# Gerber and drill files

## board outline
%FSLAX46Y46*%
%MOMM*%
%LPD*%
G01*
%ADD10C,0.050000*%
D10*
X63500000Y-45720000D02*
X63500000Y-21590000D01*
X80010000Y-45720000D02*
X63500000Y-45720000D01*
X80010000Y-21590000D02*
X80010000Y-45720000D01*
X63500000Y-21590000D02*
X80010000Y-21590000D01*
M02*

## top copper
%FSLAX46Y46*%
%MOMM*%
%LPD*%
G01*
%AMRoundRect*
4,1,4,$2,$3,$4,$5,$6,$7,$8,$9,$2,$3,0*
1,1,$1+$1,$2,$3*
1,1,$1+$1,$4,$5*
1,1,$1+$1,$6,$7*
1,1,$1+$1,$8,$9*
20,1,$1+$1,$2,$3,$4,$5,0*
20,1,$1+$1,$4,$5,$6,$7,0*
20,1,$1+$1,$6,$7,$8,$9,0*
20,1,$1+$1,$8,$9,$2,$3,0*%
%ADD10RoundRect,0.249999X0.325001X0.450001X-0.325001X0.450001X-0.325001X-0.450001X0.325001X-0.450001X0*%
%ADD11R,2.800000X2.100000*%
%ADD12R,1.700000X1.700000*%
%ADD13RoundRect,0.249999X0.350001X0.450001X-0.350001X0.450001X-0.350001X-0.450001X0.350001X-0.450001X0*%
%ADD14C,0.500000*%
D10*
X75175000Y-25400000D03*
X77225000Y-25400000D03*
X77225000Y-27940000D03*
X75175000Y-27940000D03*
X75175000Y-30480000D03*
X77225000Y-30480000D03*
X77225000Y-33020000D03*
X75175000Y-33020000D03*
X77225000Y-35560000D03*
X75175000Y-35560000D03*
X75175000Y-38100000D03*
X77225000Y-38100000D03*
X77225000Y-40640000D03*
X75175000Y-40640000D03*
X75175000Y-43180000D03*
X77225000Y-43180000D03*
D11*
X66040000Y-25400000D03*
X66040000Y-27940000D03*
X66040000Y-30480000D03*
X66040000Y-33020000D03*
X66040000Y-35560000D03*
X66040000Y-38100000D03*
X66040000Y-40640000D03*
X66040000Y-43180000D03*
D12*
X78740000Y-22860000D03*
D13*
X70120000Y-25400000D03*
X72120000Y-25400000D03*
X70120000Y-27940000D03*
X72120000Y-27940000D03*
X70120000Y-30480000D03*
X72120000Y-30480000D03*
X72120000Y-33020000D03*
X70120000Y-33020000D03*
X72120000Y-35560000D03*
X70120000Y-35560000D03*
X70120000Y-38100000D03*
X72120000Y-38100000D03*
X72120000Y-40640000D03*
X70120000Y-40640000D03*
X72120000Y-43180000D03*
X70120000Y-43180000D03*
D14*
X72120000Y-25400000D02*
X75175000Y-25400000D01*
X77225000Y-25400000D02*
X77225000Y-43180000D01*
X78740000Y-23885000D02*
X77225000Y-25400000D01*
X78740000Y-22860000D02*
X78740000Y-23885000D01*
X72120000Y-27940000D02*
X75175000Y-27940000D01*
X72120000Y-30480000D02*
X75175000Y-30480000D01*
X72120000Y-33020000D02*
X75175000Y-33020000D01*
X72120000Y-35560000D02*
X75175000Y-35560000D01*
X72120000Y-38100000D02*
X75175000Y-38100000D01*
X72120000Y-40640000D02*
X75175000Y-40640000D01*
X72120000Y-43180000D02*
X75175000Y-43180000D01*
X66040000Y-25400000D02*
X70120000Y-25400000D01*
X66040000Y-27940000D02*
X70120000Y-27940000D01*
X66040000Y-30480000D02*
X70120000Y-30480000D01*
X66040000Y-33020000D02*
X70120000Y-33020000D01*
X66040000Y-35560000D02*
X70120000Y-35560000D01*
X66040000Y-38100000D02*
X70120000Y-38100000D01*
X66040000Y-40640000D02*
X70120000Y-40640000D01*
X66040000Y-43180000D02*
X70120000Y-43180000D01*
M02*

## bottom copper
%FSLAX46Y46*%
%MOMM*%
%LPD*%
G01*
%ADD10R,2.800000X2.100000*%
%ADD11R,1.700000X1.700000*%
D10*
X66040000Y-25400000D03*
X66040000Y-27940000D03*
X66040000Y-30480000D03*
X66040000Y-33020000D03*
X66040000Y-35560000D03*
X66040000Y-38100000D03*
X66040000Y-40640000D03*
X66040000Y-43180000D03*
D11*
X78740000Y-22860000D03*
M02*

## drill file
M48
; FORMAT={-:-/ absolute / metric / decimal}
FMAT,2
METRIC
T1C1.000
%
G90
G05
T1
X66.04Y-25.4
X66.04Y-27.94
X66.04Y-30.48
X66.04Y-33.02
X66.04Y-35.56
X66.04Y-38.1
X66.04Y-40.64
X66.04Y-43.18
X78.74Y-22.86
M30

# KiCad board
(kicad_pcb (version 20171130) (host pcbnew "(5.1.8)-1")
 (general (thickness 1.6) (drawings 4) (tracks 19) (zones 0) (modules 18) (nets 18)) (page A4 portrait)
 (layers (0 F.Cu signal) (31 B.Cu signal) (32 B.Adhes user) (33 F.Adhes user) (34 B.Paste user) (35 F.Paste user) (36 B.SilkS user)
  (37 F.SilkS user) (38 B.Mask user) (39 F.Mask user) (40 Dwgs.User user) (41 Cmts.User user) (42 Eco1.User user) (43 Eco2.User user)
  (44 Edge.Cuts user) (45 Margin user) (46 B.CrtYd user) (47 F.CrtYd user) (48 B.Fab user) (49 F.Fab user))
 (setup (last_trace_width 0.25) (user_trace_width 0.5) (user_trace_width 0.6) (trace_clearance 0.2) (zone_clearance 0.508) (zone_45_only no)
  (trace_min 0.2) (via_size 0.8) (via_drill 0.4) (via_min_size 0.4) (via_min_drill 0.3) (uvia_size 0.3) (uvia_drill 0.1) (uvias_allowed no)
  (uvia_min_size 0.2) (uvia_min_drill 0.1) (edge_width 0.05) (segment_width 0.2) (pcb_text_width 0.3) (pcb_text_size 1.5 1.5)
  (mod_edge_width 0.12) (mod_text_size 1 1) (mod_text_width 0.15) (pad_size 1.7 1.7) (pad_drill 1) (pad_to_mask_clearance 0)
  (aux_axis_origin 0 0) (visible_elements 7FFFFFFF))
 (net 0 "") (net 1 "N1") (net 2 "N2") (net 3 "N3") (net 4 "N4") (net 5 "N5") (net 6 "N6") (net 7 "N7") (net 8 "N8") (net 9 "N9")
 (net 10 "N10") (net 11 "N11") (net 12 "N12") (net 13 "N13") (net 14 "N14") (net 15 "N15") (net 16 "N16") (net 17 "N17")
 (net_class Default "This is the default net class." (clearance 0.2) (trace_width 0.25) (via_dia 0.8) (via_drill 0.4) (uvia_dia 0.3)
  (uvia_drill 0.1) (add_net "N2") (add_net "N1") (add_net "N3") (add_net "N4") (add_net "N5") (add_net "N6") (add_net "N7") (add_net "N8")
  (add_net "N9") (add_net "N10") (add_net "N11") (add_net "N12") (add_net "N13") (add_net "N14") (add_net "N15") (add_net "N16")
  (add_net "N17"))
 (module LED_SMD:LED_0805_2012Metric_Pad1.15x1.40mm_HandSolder (layer F.Cu) (at 76.2 25.4 180)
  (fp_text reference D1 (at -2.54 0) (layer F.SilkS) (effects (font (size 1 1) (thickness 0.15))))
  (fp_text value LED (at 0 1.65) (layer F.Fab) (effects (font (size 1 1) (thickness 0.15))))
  (pad 2 smd roundrect (at 1.025 0 180) (size 1.15 1.4) (layers F.Cu F.Paste F.Mask) (roundrect_rratio 0.2173904347826087) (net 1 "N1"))
  (pad 1 smd roundrect (at -1.025 0 180) (size 1.15 1.4) (layers F.Cu F.Paste F.Mask) (roundrect_rratio 0.2173904347826087) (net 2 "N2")))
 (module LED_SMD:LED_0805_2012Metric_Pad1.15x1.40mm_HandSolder (layer F.Cu) (at 76.2 27.94 180)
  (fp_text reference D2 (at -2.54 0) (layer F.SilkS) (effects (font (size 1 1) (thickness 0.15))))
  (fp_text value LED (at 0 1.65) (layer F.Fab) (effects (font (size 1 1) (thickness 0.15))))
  (pad 1 smd roundrect (at -1.025 0 180) (size 1.15 1.4) (layers F.Cu F.Paste F.Mask) (roundrect_rratio 0.2173904347826087) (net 2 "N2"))
  (pad 2 smd roundrect (at 1.025 0 180) (size 1.15 1.4) (layers F.Cu F.Paste F.Mask) (roundrect_rratio 0.2173904347826087) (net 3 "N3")))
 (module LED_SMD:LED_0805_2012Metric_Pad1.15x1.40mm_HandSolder (layer F.Cu) (at 76.2 30.48 180)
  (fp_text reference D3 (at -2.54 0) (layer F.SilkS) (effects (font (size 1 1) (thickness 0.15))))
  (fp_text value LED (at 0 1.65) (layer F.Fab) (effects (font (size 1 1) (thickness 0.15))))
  (pad 2 smd roundrect (at 1.025 0 180) (size 1.15 1.4) (layers F.Cu F.Paste F.Mask) (roundrect_rratio 0.2173904347826087) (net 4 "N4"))
  (pad 1 smd roundrect (at -1.025 0 180) (size 1.15 1.4) (layers F.Cu F.Paste F.Mask) (roundrect_rratio 0.2173904347826087) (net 2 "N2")))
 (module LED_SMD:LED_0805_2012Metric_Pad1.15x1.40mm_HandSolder (layer F.Cu) (at 76.2 33.02 180)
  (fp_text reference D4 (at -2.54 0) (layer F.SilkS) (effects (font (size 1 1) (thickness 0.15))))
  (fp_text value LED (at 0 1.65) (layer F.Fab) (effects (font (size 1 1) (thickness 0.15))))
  (pad 1 smd roundrect (at -1.025 0 180) (size 1.15 1.4) (layers F.Cu F.Paste F.Mask) (roundrect_rratio 0.2173904347826087) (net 2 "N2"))
  (pad 2 smd roundrect (at 1.025 0 180) (size 1.15 1.4) (layers F.Cu F.Paste F.Mask) (roundrect_rratio 0.2173904347826087) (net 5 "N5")))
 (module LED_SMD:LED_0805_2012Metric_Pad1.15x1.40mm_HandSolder (layer F.Cu) (at 76.2 35.56 180)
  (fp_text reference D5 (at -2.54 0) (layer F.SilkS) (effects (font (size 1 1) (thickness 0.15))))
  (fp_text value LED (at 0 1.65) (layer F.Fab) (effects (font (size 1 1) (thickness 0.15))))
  (pad 1 smd roundrect (at -1.025 0 180) (size 1.15 1.4) (layers F.Cu F.Paste F.Mask) (roundrect_rratio 0.2173904347826087) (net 2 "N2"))
  (pad 2 smd roundrect (at 1.025 0 180) (size 1.15 1.4) (layers F.Cu F.Paste F.Mask) (roundrect_rratio 0.2173904347826087) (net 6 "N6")))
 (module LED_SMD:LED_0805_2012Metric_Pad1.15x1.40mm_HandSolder (layer F.Cu) (at 76.2 38.1 180)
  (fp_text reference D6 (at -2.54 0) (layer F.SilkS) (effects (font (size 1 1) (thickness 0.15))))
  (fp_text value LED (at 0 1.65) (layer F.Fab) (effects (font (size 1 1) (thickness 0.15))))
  (pad 2 smd roundrect (at 1.025 0 180) (size 1.15 1.4) (layers F.Cu F.Paste F.Mask) (roundrect_rratio 0.2173904347826087) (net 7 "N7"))
  (pad 1 smd roundrect (at -1.025 0 180) (size 1.15 1.4) (layers F.Cu F.Paste F.Mask) (roundrect_rratio 0.2173904347826087) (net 2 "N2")))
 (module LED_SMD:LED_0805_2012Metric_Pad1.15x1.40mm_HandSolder (layer F.Cu) (at 76.2 40.64 180)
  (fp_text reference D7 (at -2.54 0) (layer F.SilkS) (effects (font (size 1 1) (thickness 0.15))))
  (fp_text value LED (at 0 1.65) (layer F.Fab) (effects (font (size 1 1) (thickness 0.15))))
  (pad 1 smd roundrect (at -1.025 0 180) (size 1.15 1.4) (layers F.Cu F.Paste F.Mask) (roundrect_rratio 0.2173904347826087) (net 2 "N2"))
  (pad 2 smd roundrect (at 1.025 0 180) (size 1.15 1.4) (layers F.Cu F.Paste F.Mask) (roundrect_rratio 0.2173904347826087) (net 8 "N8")))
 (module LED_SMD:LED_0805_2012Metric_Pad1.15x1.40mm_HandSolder (layer F.Cu) (at 76.2 43.18 180)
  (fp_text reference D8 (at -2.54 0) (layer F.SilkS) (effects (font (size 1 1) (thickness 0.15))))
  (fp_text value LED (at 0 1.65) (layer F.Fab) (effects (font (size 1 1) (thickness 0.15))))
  (pad 2 smd roundrect (at 1.025 0 180) (size 1.15 1.4) (layers F.Cu F.Paste F.Mask) (roundrect_rratio 0.2173904347826087) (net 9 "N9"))
  (pad 1 smd roundrect (at -1.025 0 180) (size 1.15 1.4) (layers F.Cu F.Paste F.Mask) (roundrect_rratio 0.2173904347826087) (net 2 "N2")))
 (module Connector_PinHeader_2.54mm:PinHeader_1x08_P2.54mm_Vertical (layer F.Cu) (at 66.04 25.4)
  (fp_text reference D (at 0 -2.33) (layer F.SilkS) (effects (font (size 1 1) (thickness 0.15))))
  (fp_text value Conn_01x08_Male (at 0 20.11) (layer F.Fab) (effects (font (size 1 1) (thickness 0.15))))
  (pad 1 thru_hole rect (at 0 0) (size 2.8 2.1) (drill 1) (layers *.Cu *.Mask) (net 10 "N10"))
  (pad 2 thru_hole rect (at 0 2.54) (size 2.8 2.1) (drill 1) (layers *.Cu *.Mask) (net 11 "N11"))
  (pad 3 thru_hole rect (at 0 5.08) (size 2.8 2.1) (drill 1) (layers *.Cu *.Mask) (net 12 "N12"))
  (pad 4 thru_hole rect (at 0 7.62) (size 2.8 2.1) (drill 1) (layers *.Cu *.Mask) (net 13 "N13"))
  (pad 5 thru_hole rect (at 0 10.16) (size 2.8 2.1) (drill 1) (layers *.Cu *.Mask) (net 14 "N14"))
  (pad 6 thru_hole rect (at 0 12.7) (size 2.8 2.1) (drill 1) (layers *.Cu *.Mask) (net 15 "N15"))
  (pad 7 thru_hole rect (at 0 15.24) (size 2.8 2.1) (drill 1) (layers *.Cu *.Mask) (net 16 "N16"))
  (pad 8 thru_hole rect (at 0 17.78) (size 2.8 2.1) (drill 1) (layers *.Cu *.Mask) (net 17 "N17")))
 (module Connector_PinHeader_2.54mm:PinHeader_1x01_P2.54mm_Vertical (layer F.Cu) (at 78.74 22.86)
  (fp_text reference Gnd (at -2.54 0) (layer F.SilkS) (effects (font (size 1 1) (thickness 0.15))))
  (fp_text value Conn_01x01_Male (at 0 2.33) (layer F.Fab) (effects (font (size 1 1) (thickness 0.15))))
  (pad 1 thru_hole rect (at 0 0) (size 1.7 1.7) (drill 1) (layers *.Cu *.Mask) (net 2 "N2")))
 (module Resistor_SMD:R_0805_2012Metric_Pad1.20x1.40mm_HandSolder (layer F.Cu) (at 71.12 25.4 180)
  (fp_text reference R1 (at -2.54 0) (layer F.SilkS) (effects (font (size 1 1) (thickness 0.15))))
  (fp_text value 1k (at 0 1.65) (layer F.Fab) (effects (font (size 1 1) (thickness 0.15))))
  (pad 2 smd roundrect (at 1 0 180) (size 1.2 1.4) (layers F.Cu F.Paste F.Mask) (roundrect_rratio 0.2083325) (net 10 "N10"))
  (pad 1 smd roundrect (at -1 0 180) (size 1.2 1.4) (layers F.Cu F.Paste F.Mask) (roundrect_rratio 0.2083325) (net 1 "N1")))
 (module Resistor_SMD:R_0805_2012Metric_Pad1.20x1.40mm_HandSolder (layer F.Cu) (at 71.12 27.94 180)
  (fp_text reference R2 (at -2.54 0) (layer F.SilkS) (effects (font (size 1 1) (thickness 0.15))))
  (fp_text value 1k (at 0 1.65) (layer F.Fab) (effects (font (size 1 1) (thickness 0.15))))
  (pad 2 smd roundrect (at 1 0 180) (size 1.2 1.4) (layers F.Cu F.Paste F.Mask) (roundrect_rratio 0.2083325) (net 11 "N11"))
  (pad 1 smd roundrect (at -1 0 180) (size 1.2 1.4) (layers F.Cu F.Paste F.Mask) (roundrect_rratio 0.2083325) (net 3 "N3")))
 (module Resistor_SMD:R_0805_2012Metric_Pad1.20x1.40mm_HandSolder (layer F.Cu) (at 71.12 30.48 180)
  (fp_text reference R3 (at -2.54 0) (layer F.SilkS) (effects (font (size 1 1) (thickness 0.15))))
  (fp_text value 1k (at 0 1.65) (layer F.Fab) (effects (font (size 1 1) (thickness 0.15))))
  (pad 2 smd roundrect (at 1 0 180) (size 1.2 1.4) (layers F.Cu F.Paste F.Mask) (roundrect_rratio 0.2083325) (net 12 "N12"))
  (pad 1 smd roundrect (at -1 0 180) (size 1.2 1.4) (layers F.Cu F.Paste F.Mask) (roundrect_rratio 0.2083325) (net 4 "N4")))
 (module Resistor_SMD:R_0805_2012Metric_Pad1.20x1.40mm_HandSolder (layer F.Cu) (at 71.12 33.02 180)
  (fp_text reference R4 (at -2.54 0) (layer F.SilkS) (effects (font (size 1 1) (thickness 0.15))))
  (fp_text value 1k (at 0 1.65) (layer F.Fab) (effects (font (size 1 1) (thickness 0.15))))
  (pad 1 smd roundrect (at -1 0 180) (size 1.2 1.4) (layers F.Cu F.Paste F.Mask) (roundrect_rratio 0.2083325) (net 5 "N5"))
  (pad 2 smd roundrect (at 1 0 180) (size 1.2 1.4) (layers F.Cu F.Paste F.Mask) (roundrect_rratio 0.2083325) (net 13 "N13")))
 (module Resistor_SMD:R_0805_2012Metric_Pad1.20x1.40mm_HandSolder (layer F.Cu) (at 71.12 35.56 180)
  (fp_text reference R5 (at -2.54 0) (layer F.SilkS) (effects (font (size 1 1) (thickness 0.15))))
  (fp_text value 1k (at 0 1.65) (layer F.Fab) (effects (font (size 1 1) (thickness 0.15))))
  (pad 1 smd roundrect (at -1 0 180) (size 1.2 1.4) (layers F.Cu F.Paste F.Mask) (roundrect_rratio 0.2083325) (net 6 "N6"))
  (pad 2 smd roundrect (at 1 0 180) (size 1.2 1.4) (layers F.Cu F.Paste F.Mask) (roundrect_rratio 0.2083325) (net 14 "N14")))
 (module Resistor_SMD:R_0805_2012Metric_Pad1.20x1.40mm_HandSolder (layer F.Cu) (at 71.12 38.1 180)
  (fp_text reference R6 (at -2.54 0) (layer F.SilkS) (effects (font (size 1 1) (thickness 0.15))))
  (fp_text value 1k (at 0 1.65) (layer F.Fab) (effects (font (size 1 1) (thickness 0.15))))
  (pad 2 smd roundrect (at 1 0 180) (size 1.2 1.4) (layers F.Cu F.Paste F.Mask) (roundrect_rratio 0.2083325) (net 15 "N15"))
  (pad 1 smd roundrect (at -1 0 180) (size 1.2 1.4) (layers F.Cu F.Paste F.Mask) (roundrect_rratio 0.2083325) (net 7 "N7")))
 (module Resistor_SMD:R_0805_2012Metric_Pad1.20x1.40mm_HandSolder (layer F.Cu) (at 71.12 40.64 180)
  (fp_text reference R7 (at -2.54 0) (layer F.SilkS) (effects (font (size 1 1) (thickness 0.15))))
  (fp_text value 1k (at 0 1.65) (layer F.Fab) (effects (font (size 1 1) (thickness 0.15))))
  (pad 1 smd roundrect (at -1 0 180) (size 1.2 1.4) (layers F.Cu F.Paste F.Mask) (roundrect_rratio 0.2083325) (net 8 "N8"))
  (pad 2 smd roundrect (at 1 0 180) (size 1.2 1.4) (layers F.Cu F.Paste F.Mask) (roundrect_rratio 0.2083325) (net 16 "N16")))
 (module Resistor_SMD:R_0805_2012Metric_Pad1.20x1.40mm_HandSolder (layer F.Cu) (at 71.12 43.18 180)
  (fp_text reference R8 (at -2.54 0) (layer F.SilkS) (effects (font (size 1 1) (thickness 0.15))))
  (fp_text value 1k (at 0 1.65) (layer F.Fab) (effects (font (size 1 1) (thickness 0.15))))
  (pad 1 smd roundrect (at -1 0 180) (size 1.2 1.4) (layers F.Cu F.Paste F.Mask) (roundrect_rratio 0.2083325) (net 9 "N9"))
  (pad 2 smd roundrect (at 1 0 180) (size 1.2 1.4) (layers F.Cu F.Paste F.Mask) (roundrect_rratio 0.2083325) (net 17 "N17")))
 (gr_line (start 63.5 45.72) (end 63.5 21.59) (layer Edge.Cuts) (width 0.05))
 (gr_line (start 80.01 45.72) (end 63.5 45.72) (layer Edge.Cuts) (width 0.05))
 (gr_line (start 80.01 21.59) (end 80.01 45.72) (layer Edge.Cuts) (width 0.05))
 (gr_line (start 63.5 21.59) (end 80.01 21.59) (layer Edge.Cuts) (width 0.05))
 (segment (start 72.12 25.4) (end 75.175 25.4) (width 0.5) (layer F.Cu) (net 1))
 (segment (start 77.225 25.4) (end 77.225 43.18) (width 0.5) (layer F.Cu) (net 2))
 (segment (start 78.74 23.885) (end 77.225 25.4) (width 0.5) (layer F.Cu) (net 2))
 (segment (start 78.74 22.86) (end 78.74 23.885) (width 0.5) (layer F.Cu) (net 2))
 (segment (start 72.12 27.94) (end 75.175 27.94) (width 0.5) (layer F.Cu) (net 3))
 (segment (start 72.12 30.48) (end 75.175 30.48) (width 0.5) (layer F.Cu) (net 4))
 (segment (start 72.12 33.02) (end 75.175 33.02) (width 0.5) (layer F.Cu) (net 5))
 (segment (start 72.12 35.56) (end 75.175 35.56) (width 0.5) (layer F.Cu) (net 6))
 (segment (start 72.12 38.1) (end 75.175 38.1) (width 0.5) (layer F.Cu) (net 7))
 (segment (start 72.12 40.64) (end 75.175 40.64) (width 0.5) (layer F.Cu) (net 8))
 (segment (start 72.12 43.18) (end 75.175 43.18) (width 0.5) (layer F.Cu) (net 9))
 (segment (start 66.04 25.4) (end 70.12 25.4) (width 0.5) (layer F.Cu) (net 10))
 (segment (start 66.04 27.94) (end 70.12 27.94) (width 0.5) (layer F.Cu) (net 11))
 (segment (start 66.04 30.48) (end 70.12 30.48) (width 0.5) (layer F.Cu) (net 12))
 (segment (start 66.04 33.02) (end 70.12 33.02) (width 0.5) (layer F.Cu) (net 13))
 (segment (start 66.04 35.56) (end 70.12 35.56) (width 0.5) (layer F.Cu) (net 14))
 (segment (start 66.04 38.1) (end 70.12 38.1) (width 0.5) (layer F.Cu) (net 15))
 (segment (start 66.04 40.64) (end 70.12 40.64) (width 0.5) (layer F.Cu) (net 16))
 (segment (start 66.04 43.18) (end 70.12 43.18) (width 0.5) (layer F.Cu) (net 17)))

